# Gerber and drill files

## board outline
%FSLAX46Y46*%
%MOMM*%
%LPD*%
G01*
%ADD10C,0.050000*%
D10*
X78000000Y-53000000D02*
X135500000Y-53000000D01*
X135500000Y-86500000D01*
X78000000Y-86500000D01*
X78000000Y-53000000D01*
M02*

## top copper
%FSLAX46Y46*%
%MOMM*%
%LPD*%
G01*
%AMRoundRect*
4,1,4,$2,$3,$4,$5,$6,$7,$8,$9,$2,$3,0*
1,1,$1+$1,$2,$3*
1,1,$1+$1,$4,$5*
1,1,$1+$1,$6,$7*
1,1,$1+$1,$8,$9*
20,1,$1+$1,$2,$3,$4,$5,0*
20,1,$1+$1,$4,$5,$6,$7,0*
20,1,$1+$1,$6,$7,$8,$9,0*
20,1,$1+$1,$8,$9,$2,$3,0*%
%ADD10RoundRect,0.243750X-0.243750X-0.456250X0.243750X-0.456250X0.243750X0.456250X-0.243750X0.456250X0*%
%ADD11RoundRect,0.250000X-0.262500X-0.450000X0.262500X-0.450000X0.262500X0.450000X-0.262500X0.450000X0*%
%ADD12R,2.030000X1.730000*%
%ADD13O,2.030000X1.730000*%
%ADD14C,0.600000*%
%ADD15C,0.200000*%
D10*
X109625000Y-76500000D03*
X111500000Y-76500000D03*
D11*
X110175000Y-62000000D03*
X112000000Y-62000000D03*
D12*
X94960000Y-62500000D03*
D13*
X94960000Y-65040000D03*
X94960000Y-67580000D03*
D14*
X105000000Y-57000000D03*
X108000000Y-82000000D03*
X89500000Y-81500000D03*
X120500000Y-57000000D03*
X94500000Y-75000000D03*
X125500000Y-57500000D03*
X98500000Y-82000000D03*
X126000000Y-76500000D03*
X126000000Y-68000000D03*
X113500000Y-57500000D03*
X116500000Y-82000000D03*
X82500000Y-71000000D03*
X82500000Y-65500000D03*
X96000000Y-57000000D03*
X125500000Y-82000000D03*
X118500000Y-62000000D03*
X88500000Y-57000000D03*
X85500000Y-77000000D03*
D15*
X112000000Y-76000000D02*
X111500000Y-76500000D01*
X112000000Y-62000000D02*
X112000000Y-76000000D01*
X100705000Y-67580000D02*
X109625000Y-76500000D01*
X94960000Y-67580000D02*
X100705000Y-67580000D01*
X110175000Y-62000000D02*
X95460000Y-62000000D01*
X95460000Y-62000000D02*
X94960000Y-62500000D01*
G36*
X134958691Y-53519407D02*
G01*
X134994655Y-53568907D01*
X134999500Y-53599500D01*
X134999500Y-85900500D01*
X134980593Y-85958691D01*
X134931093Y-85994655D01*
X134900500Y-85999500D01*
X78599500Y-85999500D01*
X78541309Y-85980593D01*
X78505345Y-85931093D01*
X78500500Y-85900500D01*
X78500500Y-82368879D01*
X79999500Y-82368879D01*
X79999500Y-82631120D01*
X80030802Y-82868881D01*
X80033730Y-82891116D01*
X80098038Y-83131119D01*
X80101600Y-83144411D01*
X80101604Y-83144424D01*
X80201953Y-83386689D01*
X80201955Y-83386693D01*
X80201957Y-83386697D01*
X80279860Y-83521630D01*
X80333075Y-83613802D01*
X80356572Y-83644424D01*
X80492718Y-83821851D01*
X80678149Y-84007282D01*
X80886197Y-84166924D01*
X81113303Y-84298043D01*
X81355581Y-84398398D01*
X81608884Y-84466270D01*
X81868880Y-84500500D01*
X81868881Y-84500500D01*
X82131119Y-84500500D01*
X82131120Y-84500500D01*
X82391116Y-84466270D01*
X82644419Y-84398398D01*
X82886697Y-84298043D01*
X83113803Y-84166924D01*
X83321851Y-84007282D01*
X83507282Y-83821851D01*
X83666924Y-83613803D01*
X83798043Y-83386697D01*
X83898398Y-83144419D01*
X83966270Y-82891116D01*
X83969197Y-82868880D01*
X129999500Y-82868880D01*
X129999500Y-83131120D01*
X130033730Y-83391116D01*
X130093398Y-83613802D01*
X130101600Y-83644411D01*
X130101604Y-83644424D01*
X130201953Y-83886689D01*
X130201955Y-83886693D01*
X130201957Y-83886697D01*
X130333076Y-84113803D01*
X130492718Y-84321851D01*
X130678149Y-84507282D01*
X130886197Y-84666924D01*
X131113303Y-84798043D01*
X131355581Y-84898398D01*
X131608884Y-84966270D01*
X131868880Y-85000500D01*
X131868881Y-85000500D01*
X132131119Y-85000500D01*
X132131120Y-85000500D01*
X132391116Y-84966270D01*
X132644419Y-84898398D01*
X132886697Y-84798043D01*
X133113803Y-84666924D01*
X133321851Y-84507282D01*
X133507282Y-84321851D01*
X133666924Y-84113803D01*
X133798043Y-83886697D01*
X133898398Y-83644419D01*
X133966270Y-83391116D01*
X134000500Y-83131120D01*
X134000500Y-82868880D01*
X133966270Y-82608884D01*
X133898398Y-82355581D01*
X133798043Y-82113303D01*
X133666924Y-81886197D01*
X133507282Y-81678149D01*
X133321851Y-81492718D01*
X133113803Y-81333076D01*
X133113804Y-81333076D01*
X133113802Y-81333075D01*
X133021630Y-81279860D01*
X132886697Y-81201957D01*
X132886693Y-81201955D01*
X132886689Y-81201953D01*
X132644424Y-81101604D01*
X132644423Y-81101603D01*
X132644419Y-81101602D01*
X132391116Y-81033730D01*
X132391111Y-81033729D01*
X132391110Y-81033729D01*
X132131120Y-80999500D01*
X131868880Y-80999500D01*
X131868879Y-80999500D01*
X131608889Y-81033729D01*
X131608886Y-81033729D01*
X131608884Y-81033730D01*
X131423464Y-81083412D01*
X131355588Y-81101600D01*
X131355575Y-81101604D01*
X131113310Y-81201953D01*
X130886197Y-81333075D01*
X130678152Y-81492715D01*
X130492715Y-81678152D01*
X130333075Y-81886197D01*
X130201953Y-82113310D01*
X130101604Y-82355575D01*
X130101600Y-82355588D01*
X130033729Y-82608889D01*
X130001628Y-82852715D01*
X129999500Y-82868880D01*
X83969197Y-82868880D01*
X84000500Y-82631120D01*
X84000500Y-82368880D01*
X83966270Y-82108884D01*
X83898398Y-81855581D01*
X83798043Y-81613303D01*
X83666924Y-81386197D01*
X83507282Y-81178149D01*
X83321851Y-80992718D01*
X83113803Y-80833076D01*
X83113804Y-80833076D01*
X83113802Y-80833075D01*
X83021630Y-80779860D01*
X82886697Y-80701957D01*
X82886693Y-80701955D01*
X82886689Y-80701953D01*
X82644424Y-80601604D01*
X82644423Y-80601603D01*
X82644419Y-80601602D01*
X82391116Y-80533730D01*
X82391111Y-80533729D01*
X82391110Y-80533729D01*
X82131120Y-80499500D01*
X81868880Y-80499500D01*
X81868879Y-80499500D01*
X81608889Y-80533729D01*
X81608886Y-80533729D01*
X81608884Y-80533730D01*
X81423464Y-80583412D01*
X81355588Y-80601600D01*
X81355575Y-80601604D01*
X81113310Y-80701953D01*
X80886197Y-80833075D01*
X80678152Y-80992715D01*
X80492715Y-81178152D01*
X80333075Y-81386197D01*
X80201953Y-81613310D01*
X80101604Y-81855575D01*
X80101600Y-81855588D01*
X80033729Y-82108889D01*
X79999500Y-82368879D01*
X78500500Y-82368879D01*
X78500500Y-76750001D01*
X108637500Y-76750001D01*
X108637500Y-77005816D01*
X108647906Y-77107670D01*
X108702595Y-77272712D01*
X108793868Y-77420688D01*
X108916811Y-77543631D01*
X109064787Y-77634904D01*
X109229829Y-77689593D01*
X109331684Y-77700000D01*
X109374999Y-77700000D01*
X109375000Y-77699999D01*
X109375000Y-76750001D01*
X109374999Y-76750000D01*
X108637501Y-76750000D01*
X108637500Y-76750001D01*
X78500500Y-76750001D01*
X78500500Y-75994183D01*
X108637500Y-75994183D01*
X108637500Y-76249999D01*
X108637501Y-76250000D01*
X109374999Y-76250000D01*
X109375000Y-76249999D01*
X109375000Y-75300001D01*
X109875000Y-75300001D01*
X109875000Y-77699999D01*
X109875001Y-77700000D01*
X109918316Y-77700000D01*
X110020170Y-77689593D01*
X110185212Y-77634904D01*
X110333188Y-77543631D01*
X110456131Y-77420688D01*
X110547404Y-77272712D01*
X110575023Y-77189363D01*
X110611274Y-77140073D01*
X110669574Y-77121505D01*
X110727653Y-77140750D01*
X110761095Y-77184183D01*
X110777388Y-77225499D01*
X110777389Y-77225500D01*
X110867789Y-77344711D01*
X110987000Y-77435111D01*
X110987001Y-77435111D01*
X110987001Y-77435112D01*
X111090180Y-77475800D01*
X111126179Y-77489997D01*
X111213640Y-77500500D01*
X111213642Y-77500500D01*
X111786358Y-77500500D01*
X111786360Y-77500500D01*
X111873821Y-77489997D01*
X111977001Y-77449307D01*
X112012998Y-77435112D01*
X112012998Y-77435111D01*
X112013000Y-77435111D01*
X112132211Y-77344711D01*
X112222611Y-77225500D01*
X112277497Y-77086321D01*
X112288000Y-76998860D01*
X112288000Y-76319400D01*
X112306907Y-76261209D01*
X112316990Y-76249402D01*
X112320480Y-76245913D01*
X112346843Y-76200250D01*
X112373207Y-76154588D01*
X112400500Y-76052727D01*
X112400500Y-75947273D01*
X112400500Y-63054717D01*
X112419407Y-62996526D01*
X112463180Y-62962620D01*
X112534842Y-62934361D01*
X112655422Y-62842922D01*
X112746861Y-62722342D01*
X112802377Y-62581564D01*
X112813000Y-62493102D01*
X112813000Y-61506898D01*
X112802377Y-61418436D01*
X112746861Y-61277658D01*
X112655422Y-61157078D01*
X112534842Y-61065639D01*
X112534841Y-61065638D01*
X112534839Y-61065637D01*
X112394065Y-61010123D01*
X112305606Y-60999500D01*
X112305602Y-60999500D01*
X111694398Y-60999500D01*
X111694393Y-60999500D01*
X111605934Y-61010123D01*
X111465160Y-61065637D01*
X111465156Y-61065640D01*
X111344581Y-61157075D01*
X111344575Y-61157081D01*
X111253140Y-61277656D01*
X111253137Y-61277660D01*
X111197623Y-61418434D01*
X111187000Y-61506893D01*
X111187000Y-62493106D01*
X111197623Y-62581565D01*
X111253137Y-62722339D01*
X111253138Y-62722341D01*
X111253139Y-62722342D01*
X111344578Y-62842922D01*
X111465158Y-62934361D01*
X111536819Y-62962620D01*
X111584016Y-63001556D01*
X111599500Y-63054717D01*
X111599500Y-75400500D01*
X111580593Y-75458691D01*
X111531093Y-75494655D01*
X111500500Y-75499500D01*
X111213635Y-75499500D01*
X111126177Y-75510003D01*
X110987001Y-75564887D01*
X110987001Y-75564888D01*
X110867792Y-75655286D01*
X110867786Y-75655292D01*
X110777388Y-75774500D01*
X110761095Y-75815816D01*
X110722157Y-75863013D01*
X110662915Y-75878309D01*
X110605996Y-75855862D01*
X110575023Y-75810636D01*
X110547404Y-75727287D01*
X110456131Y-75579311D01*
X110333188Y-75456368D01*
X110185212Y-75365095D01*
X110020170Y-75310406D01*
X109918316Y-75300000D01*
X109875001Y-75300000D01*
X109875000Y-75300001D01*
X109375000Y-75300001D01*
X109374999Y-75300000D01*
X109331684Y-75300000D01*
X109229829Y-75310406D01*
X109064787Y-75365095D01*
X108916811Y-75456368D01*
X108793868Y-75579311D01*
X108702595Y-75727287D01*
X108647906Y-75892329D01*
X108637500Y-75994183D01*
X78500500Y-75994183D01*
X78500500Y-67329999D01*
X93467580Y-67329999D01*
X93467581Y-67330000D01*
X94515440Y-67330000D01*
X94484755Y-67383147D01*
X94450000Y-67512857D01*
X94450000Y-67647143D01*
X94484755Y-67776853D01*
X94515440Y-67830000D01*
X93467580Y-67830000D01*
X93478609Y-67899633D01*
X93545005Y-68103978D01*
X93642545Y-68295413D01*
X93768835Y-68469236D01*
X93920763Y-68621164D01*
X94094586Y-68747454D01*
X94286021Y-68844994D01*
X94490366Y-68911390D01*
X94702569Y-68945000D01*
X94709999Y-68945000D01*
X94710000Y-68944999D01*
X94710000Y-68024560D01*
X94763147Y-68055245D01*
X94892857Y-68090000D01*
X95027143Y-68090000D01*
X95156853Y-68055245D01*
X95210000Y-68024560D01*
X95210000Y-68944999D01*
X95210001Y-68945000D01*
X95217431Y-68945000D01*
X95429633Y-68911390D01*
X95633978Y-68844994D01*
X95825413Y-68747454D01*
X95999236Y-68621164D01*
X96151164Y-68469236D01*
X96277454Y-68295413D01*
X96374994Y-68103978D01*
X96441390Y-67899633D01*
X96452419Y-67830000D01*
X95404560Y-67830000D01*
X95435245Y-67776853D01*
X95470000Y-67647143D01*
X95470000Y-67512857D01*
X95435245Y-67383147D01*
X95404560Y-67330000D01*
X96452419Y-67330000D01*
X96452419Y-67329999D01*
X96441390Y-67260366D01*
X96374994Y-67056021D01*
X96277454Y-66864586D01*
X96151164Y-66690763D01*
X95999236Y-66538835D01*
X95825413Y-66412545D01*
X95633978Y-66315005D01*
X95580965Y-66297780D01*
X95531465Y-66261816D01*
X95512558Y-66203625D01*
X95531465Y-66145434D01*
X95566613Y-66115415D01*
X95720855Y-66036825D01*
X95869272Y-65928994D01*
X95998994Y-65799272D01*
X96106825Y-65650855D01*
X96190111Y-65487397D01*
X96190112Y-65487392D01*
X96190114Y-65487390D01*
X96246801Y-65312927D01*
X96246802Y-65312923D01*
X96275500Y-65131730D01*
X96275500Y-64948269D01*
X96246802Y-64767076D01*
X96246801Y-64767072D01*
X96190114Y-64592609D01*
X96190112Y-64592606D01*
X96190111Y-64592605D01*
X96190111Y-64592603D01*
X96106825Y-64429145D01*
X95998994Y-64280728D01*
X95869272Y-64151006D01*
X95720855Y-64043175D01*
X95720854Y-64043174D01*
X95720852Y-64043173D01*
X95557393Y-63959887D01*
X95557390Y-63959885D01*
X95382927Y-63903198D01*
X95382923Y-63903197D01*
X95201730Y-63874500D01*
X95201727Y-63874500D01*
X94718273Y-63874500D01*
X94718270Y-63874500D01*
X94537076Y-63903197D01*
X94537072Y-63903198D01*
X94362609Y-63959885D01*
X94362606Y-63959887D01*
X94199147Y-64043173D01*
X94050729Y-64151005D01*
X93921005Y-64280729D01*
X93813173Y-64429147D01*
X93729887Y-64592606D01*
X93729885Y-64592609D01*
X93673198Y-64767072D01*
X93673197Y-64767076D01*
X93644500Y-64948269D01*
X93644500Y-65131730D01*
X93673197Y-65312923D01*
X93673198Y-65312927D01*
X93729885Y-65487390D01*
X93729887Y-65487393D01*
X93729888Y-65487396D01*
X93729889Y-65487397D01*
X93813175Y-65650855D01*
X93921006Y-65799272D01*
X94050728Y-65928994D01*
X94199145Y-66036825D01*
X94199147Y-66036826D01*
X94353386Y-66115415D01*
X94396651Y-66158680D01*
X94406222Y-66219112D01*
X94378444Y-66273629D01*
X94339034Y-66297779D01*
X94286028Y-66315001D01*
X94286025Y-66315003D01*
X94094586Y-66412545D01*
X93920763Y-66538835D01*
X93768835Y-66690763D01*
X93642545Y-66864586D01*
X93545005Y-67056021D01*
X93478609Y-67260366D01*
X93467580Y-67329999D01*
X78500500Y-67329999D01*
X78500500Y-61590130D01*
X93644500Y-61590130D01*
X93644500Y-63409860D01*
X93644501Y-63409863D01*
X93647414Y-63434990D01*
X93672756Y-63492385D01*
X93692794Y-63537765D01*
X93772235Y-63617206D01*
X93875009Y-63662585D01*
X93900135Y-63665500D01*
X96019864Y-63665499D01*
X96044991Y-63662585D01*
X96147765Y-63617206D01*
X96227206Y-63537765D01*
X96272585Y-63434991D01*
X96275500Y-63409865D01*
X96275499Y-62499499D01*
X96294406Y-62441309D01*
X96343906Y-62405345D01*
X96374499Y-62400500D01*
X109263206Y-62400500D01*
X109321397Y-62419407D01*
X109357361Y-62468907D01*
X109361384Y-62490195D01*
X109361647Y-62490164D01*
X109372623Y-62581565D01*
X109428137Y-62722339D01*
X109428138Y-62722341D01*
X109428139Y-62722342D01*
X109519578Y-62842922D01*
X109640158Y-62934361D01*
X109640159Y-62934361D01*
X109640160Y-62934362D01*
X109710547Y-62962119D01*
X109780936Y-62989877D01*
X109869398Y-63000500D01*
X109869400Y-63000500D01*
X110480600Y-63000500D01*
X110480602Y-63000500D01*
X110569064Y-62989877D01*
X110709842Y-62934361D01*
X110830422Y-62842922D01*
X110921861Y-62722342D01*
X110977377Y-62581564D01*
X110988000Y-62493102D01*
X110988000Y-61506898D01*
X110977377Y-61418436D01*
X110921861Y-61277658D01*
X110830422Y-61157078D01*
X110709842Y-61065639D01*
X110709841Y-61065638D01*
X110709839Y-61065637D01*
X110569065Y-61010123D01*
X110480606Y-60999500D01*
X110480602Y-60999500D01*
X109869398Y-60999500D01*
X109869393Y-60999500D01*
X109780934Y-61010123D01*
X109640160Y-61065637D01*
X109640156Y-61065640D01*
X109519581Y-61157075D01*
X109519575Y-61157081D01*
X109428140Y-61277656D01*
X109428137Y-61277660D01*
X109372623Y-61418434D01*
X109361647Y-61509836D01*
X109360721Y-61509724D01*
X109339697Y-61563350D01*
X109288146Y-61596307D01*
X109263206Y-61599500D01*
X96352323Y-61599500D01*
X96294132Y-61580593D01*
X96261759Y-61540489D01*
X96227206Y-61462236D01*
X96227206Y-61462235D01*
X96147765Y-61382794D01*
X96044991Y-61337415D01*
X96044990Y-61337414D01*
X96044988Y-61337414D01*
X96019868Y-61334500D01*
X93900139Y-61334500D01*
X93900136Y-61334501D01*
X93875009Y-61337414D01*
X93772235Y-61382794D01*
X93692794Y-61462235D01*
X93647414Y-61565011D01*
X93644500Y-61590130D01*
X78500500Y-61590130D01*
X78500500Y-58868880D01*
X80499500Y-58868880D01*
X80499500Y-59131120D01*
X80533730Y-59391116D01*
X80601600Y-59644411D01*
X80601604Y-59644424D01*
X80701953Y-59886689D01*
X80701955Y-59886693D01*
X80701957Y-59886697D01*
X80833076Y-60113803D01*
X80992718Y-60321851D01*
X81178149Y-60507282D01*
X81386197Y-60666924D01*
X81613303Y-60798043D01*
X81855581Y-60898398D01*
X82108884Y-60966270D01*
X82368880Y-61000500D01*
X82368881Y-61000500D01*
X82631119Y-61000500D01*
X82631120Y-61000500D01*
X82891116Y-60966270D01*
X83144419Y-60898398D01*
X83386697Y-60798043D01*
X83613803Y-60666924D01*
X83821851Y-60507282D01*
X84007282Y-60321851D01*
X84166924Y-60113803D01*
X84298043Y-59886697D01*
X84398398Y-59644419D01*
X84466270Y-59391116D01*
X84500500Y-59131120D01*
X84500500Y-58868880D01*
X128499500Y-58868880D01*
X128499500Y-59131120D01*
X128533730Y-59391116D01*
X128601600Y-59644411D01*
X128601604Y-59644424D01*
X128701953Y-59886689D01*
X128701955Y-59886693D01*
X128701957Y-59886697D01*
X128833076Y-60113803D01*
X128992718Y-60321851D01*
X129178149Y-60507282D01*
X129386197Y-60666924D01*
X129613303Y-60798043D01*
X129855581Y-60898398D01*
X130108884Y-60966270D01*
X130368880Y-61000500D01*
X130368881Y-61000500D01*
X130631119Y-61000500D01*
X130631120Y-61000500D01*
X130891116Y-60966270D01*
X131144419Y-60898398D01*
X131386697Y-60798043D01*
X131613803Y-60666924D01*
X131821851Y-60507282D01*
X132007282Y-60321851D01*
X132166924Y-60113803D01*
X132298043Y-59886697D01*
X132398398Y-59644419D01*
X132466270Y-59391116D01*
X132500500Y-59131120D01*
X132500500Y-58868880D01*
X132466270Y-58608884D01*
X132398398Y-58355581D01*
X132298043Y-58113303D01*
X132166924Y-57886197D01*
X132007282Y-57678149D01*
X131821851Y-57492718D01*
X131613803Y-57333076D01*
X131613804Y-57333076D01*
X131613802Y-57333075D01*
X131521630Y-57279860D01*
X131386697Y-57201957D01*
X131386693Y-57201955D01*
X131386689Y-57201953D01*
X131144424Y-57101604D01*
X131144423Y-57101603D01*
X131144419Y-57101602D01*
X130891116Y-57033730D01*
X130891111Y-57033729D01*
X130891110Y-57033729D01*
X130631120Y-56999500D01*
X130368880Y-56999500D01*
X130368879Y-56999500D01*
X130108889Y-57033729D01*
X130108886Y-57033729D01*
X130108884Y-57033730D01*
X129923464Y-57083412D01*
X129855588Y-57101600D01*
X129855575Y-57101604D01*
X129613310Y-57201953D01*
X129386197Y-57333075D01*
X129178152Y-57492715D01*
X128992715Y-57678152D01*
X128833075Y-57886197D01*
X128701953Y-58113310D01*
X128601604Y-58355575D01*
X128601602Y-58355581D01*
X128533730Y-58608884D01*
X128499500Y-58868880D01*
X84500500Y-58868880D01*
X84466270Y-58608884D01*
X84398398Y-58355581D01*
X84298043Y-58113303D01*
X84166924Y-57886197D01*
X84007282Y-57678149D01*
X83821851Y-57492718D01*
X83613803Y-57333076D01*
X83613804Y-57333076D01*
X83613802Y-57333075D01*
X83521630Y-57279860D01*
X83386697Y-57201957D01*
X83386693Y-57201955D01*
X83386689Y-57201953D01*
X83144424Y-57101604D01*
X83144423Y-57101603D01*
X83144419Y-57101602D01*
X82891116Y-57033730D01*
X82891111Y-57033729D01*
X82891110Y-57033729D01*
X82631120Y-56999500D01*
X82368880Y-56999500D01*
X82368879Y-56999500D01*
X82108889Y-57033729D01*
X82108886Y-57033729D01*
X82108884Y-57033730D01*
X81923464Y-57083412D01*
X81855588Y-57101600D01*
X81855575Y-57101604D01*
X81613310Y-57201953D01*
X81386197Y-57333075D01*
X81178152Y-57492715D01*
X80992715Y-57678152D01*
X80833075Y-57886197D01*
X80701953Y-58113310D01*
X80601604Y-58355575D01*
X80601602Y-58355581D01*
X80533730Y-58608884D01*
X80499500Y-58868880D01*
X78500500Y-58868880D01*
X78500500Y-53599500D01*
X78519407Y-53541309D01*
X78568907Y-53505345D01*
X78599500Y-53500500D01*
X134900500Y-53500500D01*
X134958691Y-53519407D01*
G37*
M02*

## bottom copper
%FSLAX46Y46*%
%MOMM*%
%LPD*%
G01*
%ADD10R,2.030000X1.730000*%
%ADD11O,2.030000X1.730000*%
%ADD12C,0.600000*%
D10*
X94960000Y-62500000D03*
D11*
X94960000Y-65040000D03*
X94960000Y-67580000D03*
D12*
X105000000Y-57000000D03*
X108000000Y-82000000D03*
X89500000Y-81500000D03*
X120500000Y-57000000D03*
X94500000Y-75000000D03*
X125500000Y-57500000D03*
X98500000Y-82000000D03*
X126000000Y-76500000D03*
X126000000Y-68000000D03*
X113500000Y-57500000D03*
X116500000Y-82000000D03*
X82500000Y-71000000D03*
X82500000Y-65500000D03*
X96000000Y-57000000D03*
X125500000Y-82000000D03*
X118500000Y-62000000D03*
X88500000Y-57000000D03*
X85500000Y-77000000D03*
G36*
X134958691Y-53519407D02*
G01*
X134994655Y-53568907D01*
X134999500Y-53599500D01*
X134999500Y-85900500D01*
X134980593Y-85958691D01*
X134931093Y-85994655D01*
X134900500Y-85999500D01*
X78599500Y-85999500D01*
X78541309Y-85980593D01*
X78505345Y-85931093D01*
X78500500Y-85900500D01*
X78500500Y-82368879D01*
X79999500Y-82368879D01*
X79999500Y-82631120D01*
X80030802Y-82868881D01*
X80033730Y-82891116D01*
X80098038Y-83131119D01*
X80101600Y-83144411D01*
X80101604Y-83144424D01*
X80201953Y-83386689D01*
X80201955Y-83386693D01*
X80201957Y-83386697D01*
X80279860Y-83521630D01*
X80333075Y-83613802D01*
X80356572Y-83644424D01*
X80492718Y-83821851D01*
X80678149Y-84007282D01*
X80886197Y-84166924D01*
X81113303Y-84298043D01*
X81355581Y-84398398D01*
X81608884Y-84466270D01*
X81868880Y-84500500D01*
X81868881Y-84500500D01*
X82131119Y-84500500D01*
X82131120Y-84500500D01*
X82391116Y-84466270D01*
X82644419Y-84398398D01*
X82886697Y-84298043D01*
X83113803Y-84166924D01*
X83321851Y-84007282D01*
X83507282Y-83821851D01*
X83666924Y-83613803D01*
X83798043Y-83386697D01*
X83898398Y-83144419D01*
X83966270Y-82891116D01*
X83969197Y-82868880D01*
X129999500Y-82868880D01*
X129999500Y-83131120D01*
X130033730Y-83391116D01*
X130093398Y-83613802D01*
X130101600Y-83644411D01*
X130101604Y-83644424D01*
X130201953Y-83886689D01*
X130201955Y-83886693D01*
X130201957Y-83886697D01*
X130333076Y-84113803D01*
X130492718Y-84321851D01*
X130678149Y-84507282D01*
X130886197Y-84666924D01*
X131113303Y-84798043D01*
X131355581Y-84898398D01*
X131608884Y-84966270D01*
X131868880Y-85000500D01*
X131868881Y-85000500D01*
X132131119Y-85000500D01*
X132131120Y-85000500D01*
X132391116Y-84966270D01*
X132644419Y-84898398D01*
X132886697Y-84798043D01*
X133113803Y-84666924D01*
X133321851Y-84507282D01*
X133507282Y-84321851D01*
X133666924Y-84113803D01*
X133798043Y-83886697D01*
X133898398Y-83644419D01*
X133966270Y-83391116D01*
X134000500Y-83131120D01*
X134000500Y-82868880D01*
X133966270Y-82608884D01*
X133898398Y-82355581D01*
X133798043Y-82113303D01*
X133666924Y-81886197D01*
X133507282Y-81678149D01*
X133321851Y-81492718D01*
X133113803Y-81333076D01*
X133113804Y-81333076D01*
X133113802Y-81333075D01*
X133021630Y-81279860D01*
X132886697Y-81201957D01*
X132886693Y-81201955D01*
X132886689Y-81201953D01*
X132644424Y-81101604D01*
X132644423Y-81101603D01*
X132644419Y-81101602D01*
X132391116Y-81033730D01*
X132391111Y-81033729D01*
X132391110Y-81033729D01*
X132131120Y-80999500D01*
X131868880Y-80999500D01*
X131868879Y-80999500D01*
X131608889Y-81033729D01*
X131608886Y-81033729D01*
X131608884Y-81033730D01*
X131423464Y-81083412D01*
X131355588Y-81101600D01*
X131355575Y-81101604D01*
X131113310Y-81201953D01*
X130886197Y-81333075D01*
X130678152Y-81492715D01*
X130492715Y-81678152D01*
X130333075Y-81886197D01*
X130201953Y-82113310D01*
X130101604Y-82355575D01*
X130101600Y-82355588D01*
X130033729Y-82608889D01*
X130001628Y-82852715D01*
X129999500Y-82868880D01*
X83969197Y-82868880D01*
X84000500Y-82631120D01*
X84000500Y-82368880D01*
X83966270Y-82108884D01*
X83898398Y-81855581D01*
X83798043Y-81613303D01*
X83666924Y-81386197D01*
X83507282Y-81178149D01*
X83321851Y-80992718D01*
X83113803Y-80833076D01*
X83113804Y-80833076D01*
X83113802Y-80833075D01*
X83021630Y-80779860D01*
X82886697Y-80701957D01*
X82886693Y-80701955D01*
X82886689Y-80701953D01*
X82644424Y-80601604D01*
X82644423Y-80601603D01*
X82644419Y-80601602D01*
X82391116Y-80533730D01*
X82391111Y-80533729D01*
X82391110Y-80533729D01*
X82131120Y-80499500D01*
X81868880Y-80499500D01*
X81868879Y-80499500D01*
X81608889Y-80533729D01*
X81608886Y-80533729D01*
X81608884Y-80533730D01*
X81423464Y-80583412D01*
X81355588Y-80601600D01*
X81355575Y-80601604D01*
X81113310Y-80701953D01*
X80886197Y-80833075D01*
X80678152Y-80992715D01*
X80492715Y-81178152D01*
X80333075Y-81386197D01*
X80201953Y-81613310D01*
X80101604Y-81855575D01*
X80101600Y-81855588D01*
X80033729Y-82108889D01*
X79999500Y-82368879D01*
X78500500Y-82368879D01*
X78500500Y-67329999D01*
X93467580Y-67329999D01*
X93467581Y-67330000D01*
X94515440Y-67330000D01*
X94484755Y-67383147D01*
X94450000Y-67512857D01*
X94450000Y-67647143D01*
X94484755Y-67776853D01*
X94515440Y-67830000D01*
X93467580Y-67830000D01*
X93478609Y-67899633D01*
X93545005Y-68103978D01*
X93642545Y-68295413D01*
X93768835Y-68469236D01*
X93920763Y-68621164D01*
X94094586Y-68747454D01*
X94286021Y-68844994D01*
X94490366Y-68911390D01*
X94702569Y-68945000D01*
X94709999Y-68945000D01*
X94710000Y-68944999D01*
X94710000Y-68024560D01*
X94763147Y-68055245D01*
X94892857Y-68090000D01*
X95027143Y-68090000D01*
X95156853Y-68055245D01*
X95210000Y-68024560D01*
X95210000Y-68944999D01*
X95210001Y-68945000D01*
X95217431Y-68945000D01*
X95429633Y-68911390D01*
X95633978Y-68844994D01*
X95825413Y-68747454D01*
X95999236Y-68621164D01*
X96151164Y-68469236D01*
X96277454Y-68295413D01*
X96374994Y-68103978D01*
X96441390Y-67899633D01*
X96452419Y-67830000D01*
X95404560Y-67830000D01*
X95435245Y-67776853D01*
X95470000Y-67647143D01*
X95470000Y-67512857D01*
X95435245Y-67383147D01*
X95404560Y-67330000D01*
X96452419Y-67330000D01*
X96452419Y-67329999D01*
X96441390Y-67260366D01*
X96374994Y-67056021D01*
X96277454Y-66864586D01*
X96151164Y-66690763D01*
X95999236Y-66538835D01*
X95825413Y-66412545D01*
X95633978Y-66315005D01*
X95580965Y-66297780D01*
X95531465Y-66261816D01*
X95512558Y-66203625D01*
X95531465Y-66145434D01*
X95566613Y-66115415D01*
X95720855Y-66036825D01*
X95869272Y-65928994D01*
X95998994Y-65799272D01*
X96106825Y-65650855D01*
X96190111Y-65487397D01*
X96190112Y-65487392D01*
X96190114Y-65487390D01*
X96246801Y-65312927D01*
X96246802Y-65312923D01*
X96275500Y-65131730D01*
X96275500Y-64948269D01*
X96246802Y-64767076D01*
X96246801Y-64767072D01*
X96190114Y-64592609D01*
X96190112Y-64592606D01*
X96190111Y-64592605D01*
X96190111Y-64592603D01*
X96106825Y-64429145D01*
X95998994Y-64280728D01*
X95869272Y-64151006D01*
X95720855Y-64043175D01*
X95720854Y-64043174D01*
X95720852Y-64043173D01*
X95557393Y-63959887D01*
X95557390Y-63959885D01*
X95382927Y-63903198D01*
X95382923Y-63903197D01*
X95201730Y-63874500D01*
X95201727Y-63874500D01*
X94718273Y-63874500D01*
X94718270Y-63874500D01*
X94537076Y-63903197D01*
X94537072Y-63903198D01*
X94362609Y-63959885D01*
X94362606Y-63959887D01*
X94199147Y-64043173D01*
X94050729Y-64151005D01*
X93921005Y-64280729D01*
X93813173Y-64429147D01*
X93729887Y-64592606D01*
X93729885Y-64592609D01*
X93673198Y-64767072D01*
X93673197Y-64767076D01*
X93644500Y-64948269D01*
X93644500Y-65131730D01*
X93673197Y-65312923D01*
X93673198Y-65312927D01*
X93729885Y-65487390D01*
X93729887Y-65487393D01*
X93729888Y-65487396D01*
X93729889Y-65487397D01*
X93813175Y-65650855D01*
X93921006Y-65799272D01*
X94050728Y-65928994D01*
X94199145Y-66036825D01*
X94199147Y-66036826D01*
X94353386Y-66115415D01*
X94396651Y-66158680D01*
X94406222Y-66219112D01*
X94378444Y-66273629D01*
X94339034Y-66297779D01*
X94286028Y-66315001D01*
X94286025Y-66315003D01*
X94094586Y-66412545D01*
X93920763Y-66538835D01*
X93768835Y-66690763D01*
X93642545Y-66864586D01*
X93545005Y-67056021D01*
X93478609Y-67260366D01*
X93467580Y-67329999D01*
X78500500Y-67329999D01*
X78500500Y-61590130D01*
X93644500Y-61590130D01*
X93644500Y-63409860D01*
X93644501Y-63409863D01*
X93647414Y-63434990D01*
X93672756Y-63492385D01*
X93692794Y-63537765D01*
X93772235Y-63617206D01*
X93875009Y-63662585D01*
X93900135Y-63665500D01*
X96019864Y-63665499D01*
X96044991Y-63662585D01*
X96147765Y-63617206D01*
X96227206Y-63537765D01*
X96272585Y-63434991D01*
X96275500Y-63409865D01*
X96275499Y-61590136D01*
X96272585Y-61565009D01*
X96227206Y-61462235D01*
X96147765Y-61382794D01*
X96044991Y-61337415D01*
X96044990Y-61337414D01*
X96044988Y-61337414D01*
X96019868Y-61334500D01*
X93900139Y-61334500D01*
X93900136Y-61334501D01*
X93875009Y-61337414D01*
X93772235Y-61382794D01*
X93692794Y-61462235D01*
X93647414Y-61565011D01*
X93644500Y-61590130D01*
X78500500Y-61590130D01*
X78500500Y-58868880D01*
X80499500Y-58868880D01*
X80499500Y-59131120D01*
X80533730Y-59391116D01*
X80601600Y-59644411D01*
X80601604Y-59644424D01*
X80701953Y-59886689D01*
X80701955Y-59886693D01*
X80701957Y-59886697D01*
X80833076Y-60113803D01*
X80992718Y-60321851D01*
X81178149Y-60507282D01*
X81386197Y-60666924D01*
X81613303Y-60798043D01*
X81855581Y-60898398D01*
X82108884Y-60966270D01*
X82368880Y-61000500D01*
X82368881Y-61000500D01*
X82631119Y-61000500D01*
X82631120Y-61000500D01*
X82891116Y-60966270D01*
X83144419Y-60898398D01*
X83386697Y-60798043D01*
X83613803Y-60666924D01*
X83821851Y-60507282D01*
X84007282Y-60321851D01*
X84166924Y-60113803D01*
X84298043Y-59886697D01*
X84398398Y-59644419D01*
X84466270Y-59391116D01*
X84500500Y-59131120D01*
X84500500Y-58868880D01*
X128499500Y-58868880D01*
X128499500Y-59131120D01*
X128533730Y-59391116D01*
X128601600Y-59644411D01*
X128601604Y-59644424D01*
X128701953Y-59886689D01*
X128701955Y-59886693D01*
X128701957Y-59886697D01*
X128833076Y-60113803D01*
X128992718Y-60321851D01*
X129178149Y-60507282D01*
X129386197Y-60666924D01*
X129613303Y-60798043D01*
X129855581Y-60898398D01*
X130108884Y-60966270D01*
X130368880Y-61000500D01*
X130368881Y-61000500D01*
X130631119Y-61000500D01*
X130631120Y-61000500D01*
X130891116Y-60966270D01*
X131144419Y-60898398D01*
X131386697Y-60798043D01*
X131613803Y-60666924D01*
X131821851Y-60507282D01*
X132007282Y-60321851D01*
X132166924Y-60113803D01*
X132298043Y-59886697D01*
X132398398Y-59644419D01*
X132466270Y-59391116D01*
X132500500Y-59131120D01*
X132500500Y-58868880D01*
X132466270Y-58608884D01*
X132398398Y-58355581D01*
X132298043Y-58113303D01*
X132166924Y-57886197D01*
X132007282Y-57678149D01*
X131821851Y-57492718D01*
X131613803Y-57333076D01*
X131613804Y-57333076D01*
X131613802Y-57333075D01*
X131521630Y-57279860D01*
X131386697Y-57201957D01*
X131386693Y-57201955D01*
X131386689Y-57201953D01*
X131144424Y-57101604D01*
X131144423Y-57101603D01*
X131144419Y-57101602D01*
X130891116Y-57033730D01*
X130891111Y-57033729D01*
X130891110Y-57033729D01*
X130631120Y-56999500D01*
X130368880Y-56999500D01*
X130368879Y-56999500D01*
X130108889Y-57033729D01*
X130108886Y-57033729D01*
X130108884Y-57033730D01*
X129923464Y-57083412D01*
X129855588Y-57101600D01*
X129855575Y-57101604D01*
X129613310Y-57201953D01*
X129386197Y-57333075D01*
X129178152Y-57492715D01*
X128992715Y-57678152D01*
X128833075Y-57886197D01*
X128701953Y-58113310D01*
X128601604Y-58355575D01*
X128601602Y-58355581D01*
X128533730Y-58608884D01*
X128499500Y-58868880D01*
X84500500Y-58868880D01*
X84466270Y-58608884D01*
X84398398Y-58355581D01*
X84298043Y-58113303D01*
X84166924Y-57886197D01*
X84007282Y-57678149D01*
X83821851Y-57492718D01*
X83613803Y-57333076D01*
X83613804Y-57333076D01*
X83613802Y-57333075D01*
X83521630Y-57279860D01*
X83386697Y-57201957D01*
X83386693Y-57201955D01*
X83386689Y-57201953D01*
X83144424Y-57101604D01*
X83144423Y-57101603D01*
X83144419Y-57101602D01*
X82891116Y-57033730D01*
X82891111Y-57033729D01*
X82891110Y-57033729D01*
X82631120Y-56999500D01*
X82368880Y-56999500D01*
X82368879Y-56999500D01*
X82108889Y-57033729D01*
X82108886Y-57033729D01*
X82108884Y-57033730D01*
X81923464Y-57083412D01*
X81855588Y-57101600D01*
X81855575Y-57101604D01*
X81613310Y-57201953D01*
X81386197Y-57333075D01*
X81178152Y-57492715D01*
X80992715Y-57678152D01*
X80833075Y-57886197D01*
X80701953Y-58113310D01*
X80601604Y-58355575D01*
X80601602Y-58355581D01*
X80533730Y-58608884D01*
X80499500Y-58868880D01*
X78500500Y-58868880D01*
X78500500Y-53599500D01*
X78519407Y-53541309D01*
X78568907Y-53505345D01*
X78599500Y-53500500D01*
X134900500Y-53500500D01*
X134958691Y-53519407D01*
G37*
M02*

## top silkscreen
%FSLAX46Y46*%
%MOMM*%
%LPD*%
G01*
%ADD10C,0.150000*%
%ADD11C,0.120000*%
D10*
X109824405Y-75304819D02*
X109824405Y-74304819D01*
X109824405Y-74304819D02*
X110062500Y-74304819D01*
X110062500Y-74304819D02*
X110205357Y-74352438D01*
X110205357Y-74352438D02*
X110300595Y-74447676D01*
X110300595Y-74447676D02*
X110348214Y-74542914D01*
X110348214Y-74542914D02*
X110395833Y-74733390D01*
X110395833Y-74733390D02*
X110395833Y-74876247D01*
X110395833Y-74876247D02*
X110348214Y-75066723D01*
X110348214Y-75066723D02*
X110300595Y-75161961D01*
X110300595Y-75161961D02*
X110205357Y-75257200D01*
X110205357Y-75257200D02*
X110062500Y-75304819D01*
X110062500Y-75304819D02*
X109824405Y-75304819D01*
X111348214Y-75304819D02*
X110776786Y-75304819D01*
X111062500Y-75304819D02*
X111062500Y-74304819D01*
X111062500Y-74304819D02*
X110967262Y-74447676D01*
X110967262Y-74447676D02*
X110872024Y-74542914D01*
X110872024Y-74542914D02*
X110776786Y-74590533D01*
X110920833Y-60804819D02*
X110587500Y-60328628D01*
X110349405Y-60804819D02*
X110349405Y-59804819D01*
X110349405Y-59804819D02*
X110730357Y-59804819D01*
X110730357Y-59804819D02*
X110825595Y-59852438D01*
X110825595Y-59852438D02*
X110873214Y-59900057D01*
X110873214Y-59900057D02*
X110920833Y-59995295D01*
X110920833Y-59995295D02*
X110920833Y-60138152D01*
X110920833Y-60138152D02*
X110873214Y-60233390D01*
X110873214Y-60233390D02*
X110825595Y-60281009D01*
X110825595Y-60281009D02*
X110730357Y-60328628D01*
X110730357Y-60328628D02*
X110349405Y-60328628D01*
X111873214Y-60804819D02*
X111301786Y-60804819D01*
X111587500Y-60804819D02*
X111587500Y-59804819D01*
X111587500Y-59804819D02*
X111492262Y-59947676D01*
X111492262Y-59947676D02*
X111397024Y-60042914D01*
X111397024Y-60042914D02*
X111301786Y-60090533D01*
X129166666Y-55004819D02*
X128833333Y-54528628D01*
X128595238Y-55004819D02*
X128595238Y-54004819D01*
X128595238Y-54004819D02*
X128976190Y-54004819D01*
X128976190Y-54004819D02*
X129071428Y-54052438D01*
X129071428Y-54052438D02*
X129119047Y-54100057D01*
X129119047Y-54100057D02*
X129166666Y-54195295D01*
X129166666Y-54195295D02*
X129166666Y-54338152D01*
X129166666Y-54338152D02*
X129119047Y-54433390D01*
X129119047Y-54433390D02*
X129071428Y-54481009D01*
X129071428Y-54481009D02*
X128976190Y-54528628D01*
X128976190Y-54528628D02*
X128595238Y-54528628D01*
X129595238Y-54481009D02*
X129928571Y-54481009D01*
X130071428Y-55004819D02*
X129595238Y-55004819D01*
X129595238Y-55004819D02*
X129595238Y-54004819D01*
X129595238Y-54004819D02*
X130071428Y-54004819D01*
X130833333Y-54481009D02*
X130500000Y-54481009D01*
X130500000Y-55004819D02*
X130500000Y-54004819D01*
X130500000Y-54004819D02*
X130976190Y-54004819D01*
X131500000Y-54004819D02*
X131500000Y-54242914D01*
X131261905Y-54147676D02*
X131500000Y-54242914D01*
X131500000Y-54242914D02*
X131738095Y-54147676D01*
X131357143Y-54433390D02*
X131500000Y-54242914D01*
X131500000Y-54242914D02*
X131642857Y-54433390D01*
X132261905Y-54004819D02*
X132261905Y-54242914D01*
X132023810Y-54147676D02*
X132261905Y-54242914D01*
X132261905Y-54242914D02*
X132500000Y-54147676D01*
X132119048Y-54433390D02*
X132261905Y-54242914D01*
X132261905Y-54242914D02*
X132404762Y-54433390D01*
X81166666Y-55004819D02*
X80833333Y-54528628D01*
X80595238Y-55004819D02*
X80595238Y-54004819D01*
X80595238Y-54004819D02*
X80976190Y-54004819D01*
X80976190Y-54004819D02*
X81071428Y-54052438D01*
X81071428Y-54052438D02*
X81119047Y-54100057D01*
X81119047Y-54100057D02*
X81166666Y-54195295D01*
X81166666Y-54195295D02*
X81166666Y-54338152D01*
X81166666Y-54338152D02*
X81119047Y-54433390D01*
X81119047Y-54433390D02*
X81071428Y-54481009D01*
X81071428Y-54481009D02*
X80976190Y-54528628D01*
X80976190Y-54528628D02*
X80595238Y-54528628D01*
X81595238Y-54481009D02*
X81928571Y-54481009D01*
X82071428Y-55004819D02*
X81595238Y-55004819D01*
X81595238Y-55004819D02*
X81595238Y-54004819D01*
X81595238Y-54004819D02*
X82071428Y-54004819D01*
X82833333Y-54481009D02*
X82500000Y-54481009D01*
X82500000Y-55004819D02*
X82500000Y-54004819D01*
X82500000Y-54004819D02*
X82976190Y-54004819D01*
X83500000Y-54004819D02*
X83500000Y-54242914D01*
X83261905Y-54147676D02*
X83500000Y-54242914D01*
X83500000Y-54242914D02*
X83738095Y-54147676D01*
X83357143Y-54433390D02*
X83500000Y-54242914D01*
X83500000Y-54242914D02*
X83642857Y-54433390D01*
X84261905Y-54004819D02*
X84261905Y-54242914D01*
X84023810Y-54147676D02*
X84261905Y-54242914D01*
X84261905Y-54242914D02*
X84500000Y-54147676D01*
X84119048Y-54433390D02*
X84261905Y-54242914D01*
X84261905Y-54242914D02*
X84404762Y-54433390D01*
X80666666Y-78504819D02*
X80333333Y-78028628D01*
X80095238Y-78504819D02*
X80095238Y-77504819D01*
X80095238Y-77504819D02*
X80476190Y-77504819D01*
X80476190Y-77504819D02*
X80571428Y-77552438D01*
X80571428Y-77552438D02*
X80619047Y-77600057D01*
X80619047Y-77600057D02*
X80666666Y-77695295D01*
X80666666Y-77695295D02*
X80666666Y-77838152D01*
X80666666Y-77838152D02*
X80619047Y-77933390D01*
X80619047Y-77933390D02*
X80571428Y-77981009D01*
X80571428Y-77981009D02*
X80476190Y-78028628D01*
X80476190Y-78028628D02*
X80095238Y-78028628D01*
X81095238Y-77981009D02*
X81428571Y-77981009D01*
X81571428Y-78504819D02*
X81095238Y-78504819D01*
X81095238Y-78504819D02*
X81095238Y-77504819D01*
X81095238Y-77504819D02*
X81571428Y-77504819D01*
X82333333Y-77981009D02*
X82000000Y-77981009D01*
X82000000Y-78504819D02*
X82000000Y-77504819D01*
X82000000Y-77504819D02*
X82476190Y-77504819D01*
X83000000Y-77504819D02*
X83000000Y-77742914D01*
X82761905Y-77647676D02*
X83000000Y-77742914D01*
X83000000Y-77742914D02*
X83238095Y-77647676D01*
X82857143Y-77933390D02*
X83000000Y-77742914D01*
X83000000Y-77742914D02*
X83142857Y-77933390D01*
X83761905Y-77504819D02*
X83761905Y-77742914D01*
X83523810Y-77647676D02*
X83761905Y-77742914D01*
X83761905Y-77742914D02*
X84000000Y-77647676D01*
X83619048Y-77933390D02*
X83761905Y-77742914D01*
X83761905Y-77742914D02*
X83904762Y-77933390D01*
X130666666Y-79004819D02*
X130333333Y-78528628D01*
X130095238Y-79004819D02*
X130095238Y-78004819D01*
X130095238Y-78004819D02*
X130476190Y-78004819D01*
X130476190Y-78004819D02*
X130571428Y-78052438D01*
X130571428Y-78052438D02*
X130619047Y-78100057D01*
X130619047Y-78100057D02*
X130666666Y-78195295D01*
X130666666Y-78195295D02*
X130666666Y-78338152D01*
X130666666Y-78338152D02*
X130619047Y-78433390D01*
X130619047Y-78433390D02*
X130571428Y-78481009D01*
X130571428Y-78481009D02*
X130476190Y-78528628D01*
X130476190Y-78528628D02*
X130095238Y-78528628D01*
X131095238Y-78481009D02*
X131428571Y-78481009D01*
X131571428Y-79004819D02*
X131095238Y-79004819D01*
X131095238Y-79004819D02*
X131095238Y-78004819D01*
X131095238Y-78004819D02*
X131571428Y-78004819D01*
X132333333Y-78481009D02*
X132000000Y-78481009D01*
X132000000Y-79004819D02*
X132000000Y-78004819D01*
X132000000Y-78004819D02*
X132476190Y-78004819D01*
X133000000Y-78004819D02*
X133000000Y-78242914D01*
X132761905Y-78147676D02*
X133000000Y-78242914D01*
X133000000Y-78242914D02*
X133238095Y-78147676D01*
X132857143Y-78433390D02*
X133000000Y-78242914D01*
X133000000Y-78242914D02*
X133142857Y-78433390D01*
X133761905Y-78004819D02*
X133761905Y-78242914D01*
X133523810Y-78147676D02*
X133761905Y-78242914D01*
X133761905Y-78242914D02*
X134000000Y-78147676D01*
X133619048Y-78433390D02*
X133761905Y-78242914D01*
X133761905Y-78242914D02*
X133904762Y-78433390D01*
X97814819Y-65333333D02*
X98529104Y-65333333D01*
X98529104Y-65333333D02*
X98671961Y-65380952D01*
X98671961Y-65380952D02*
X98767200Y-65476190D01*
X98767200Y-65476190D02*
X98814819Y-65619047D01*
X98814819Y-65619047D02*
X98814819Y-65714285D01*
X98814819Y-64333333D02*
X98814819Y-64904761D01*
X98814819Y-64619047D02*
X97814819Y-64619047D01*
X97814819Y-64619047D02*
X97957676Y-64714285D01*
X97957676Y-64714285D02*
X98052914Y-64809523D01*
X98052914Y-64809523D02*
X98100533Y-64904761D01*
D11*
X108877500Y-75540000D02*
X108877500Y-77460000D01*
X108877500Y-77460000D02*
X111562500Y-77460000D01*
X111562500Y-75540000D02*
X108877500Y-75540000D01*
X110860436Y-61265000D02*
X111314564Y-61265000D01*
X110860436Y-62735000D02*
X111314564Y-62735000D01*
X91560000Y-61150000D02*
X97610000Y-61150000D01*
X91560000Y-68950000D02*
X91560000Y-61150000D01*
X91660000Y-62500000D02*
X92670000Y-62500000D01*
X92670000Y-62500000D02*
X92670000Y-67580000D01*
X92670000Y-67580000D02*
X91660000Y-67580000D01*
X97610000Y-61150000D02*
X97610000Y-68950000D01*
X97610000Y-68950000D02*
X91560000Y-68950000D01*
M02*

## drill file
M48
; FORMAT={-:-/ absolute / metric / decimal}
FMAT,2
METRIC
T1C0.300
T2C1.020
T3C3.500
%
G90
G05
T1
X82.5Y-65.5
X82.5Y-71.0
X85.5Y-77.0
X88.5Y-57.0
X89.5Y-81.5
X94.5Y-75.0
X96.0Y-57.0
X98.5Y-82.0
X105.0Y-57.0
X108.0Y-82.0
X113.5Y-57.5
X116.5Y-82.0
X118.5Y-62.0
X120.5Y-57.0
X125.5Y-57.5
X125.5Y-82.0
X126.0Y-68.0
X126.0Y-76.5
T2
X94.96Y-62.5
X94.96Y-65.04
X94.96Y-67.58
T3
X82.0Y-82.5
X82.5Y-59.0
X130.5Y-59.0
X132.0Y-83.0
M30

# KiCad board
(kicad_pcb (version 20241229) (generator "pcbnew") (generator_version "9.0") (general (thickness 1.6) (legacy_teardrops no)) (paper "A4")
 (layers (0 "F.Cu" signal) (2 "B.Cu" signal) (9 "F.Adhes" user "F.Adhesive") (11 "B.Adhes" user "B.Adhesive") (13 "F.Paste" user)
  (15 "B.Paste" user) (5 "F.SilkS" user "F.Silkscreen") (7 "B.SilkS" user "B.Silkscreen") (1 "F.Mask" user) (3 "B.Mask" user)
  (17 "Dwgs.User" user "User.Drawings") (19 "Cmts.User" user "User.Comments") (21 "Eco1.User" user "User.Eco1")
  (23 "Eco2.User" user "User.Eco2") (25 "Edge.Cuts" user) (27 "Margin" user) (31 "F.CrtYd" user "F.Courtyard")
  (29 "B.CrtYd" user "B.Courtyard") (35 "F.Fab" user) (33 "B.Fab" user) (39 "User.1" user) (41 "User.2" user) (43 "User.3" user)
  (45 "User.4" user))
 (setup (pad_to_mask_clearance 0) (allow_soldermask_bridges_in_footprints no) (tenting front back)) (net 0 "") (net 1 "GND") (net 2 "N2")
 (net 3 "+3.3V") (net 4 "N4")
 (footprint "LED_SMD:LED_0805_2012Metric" (layer "F.Cu") (at 110.5625 76.5)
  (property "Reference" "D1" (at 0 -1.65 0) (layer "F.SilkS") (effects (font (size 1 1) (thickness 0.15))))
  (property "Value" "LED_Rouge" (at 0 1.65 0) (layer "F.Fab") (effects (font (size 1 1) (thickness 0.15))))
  (fp_line (start -1.685 -0.96) (end -1.685 0.96) (stroke (width 0.12) (type solid)) (layer "F.SilkS"))
  (fp_line (start -1.685 0.96) (end 1 0.96) (stroke (width 0.12) (type solid)) (layer "F.SilkS"))
  (fp_line (start 1 -0.96) (end -1.685 -0.96) (stroke (width 0.12) (type solid)) (layer "F.SilkS"))
  (pad "1" smd roundrect (at -0.9375 0) (size 0.975 1.4) (layers "F.Cu" "F.Mask" "F.Paste") (roundrect_rratio 0.25) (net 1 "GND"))
  (pad "2" smd roundrect (at 0.9375 0) (size 0.975 1.4) (layers "F.Cu" "F.Mask" "F.Paste") (roundrect_rratio 0.25) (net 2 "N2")))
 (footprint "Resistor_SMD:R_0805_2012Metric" (layer "F.Cu") (at 111.0875 62)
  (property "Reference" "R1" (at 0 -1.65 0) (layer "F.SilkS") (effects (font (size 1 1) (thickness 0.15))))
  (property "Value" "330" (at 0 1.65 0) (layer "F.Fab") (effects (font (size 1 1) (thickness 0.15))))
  (fp_line (start -0.227064 -0.735) (end 0.227064 -0.735) (stroke (width 0.12) (type solid)) (layer "F.SilkS"))
  (fp_line (start -0.227064 0.735) (end 0.227064 0.735) (stroke (width 0.12) (type solid)) (layer "F.SilkS"))
  (pad "1" smd roundrect (at -0.9125 0) (size 1.025 1.4) (layers "F.Cu" "F.Mask" "F.Paste") (roundrect_rratio 0.243902) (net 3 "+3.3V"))
  (pad "2" smd roundrect (at 0.9125 0) (size 1.025 1.4) (layers "F.Cu" "F.Mask" "F.Paste") (roundrect_rratio 0.243902) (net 2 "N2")))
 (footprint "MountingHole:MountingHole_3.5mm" (layer "F.Cu") (at 130.5 59)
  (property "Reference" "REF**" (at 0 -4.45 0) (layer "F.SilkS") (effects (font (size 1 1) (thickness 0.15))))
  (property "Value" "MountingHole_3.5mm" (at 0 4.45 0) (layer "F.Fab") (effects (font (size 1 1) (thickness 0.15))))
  (pad "" np_thru_hole circle (at 0 0) (size 3.5 3.5) (drill 3.5) (layers "*.Cu" "*.Mask")))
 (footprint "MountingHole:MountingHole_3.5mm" (layer "F.Cu") (at 82.5 59)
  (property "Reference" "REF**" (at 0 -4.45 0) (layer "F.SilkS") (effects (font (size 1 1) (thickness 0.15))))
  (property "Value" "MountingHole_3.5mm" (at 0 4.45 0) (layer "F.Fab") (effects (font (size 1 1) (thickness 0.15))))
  (pad "" np_thru_hole circle (at 0 0) (size 3.5 3.5) (drill 3.5) (layers "*.Cu" "*.Mask")))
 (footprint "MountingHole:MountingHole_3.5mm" (layer "F.Cu") (at 82 82.5)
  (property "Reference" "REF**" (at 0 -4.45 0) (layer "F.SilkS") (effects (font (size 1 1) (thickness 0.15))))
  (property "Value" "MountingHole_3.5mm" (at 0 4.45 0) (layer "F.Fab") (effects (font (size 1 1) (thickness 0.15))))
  (pad "" np_thru_hole circle (at 0 0) (size 3.5 3.5) (drill 3.5) (layers "*.Cu" "*.Mask")))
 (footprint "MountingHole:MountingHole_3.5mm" (layer "F.Cu") (at 132 83)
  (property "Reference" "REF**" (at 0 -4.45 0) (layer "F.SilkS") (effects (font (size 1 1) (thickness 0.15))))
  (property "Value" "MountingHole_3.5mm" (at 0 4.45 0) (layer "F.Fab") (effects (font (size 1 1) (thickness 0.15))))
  (pad "" np_thru_hole circle (at 0 0) (size 3.5 3.5) (drill 3.5) (layers "*.Cu" "*.Mask")))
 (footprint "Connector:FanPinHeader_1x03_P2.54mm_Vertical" (layer "F.Cu") (at 94.96 62.5 -90)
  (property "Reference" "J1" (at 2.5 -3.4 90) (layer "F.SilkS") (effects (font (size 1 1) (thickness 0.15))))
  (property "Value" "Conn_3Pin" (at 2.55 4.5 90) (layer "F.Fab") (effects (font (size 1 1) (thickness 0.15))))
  (fp_line (start -1.35 3.4) (end -1.35 -2.65) (stroke (width 0.12) (type solid)) (layer "F.SilkS"))
  (fp_line (start 6.45 3.4) (end -1.35 3.4) (stroke (width 0.12) (type solid)) (layer "F.SilkS"))
  (fp_line (start 0 3.3) (end 0 2.29) (stroke (width 0.12) (type solid)) (layer "F.SilkS"))
  (fp_line (start 0 2.29) (end 5.08 2.29) (stroke (width 0.12) (type solid)) (layer "F.SilkS"))
  (fp_line (start 5.08 2.29) (end 5.08 3.3) (stroke (width 0.12) (type solid)) (layer "F.SilkS"))
  (fp_line (start -1.35 -2.65) (end 6.45 -2.65) (stroke (width 0.12) (type solid)) (layer "F.SilkS"))
  (fp_line (start 6.45 -2.65) (end 6.45 3.4) (stroke (width 0.12) (type solid)) (layer "F.SilkS"))
  (pad "1" thru_hole rect (at 0 0) (size 2.03 1.73) (drill 1.02) (layers "*.Cu" "*.Mask") (remove_unused_layers no) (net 3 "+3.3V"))
  (pad "2" thru_hole oval (at 2.54 0) (size 2.03 1.73) (drill 1.02) (layers "*.Cu" "*.Mask") (remove_unused_layers no) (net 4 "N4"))
  (pad "3" thru_hole oval (at 5.08 0) (size 2.03 1.73) (drill 1.02) (layers "*.Cu" "*.Mask") (remove_unused_layers no) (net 1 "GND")))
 (gr_rect (start 78 53) (end 135.5 86.5) (stroke (width 0.05) (type default)) (fill no) (layer "Edge.Cuts"))
 (segment (start 112 76) (end 111.5 76.5) (width 0.2) (layer "F.Cu") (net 2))
 (segment (start 112 62) (end 112 76) (width 0.2) (layer "F.Cu") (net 2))
 (segment (start 100.705 67.58) (end 109.625 76.5) (width 0.2) (layer "F.Cu") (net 1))
 (segment (start 94.96 67.58) (end 100.705 67.58) (width 0.2) (layer "F.Cu") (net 1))
 (via (at 105 57) (size 0.6) (drill 0.3) (layers "F.Cu" "B.Cu") (free yes) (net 1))
 (via (at 108 82) (size 0.6) (drill 0.3) (layers "F.Cu" "B.Cu") (free yes) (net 1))
 (via (at 89.5 81.5) (size 0.6) (drill 0.3) (layers "F.Cu" "B.Cu") (free yes) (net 1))
 (via (at 120.5 57) (size 0.6) (drill 0.3) (layers "F.Cu" "B.Cu") (free yes) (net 1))
 (via (at 94.5 75) (size 0.6) (drill 0.3) (layers "F.Cu" "B.Cu") (free yes) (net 1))
 (via (at 125.5 57.5) (size 0.6) (drill 0.3) (layers "F.Cu" "B.Cu") (free yes) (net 1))
 (via (at 98.5 82) (size 0.6) (drill 0.3) (layers "F.Cu" "B.Cu") (free yes) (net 1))
 (via (at 126 76.5) (size 0.6) (drill 0.3) (layers "F.Cu" "B.Cu") (free yes) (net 1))
 (via (at 126 68) (size 0.6) (drill 0.3) (layers "F.Cu" "B.Cu") (free yes) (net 1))
 (via (at 113.5 57.5) (size 0.6) (drill 0.3) (layers "F.Cu" "B.Cu") (free yes) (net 1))
 (via (at 116.5 82) (size 0.6) (drill 0.3) (layers "F.Cu" "B.Cu") (free yes) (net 1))
 (via (at 82.5 71) (size 0.6) (drill 0.3) (layers "F.Cu" "B.Cu") (free yes) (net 1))
 (via (at 82.5 65.5) (size 0.6) (drill 0.3) (layers "F.Cu" "B.Cu") (free yes) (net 1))
 (via (at 96 57) (size 0.6) (drill 0.3) (layers "F.Cu" "B.Cu") (free yes) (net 1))
 (via (at 125.5 82) (size 0.6) (drill 0.3) (layers "F.Cu" "B.Cu") (free yes) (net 1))
 (via (at 118.5 62) (size 0.6) (drill 0.3) (layers "F.Cu" "B.Cu") (free yes) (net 1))
 (via (at 88.5 57) (size 0.6) (drill 0.3) (layers "F.Cu" "B.Cu") (free yes) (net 1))
 (via (at 85.5 77) (size 0.6) (drill 0.3) (layers "F.Cu" "B.Cu") (free yes) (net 1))
 (segment (start 110.175 62) (end 95.46 62) (width 0.2) (layer "F.Cu") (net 3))
 (segment (start 95.46 62) (end 94.96 62.5) (width 0.2) (layer "F.Cu") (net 3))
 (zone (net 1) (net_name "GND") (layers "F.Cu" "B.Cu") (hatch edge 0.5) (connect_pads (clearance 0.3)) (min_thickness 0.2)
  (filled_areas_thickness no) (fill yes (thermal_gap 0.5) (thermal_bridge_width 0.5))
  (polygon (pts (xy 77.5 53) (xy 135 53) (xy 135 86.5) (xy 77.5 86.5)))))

